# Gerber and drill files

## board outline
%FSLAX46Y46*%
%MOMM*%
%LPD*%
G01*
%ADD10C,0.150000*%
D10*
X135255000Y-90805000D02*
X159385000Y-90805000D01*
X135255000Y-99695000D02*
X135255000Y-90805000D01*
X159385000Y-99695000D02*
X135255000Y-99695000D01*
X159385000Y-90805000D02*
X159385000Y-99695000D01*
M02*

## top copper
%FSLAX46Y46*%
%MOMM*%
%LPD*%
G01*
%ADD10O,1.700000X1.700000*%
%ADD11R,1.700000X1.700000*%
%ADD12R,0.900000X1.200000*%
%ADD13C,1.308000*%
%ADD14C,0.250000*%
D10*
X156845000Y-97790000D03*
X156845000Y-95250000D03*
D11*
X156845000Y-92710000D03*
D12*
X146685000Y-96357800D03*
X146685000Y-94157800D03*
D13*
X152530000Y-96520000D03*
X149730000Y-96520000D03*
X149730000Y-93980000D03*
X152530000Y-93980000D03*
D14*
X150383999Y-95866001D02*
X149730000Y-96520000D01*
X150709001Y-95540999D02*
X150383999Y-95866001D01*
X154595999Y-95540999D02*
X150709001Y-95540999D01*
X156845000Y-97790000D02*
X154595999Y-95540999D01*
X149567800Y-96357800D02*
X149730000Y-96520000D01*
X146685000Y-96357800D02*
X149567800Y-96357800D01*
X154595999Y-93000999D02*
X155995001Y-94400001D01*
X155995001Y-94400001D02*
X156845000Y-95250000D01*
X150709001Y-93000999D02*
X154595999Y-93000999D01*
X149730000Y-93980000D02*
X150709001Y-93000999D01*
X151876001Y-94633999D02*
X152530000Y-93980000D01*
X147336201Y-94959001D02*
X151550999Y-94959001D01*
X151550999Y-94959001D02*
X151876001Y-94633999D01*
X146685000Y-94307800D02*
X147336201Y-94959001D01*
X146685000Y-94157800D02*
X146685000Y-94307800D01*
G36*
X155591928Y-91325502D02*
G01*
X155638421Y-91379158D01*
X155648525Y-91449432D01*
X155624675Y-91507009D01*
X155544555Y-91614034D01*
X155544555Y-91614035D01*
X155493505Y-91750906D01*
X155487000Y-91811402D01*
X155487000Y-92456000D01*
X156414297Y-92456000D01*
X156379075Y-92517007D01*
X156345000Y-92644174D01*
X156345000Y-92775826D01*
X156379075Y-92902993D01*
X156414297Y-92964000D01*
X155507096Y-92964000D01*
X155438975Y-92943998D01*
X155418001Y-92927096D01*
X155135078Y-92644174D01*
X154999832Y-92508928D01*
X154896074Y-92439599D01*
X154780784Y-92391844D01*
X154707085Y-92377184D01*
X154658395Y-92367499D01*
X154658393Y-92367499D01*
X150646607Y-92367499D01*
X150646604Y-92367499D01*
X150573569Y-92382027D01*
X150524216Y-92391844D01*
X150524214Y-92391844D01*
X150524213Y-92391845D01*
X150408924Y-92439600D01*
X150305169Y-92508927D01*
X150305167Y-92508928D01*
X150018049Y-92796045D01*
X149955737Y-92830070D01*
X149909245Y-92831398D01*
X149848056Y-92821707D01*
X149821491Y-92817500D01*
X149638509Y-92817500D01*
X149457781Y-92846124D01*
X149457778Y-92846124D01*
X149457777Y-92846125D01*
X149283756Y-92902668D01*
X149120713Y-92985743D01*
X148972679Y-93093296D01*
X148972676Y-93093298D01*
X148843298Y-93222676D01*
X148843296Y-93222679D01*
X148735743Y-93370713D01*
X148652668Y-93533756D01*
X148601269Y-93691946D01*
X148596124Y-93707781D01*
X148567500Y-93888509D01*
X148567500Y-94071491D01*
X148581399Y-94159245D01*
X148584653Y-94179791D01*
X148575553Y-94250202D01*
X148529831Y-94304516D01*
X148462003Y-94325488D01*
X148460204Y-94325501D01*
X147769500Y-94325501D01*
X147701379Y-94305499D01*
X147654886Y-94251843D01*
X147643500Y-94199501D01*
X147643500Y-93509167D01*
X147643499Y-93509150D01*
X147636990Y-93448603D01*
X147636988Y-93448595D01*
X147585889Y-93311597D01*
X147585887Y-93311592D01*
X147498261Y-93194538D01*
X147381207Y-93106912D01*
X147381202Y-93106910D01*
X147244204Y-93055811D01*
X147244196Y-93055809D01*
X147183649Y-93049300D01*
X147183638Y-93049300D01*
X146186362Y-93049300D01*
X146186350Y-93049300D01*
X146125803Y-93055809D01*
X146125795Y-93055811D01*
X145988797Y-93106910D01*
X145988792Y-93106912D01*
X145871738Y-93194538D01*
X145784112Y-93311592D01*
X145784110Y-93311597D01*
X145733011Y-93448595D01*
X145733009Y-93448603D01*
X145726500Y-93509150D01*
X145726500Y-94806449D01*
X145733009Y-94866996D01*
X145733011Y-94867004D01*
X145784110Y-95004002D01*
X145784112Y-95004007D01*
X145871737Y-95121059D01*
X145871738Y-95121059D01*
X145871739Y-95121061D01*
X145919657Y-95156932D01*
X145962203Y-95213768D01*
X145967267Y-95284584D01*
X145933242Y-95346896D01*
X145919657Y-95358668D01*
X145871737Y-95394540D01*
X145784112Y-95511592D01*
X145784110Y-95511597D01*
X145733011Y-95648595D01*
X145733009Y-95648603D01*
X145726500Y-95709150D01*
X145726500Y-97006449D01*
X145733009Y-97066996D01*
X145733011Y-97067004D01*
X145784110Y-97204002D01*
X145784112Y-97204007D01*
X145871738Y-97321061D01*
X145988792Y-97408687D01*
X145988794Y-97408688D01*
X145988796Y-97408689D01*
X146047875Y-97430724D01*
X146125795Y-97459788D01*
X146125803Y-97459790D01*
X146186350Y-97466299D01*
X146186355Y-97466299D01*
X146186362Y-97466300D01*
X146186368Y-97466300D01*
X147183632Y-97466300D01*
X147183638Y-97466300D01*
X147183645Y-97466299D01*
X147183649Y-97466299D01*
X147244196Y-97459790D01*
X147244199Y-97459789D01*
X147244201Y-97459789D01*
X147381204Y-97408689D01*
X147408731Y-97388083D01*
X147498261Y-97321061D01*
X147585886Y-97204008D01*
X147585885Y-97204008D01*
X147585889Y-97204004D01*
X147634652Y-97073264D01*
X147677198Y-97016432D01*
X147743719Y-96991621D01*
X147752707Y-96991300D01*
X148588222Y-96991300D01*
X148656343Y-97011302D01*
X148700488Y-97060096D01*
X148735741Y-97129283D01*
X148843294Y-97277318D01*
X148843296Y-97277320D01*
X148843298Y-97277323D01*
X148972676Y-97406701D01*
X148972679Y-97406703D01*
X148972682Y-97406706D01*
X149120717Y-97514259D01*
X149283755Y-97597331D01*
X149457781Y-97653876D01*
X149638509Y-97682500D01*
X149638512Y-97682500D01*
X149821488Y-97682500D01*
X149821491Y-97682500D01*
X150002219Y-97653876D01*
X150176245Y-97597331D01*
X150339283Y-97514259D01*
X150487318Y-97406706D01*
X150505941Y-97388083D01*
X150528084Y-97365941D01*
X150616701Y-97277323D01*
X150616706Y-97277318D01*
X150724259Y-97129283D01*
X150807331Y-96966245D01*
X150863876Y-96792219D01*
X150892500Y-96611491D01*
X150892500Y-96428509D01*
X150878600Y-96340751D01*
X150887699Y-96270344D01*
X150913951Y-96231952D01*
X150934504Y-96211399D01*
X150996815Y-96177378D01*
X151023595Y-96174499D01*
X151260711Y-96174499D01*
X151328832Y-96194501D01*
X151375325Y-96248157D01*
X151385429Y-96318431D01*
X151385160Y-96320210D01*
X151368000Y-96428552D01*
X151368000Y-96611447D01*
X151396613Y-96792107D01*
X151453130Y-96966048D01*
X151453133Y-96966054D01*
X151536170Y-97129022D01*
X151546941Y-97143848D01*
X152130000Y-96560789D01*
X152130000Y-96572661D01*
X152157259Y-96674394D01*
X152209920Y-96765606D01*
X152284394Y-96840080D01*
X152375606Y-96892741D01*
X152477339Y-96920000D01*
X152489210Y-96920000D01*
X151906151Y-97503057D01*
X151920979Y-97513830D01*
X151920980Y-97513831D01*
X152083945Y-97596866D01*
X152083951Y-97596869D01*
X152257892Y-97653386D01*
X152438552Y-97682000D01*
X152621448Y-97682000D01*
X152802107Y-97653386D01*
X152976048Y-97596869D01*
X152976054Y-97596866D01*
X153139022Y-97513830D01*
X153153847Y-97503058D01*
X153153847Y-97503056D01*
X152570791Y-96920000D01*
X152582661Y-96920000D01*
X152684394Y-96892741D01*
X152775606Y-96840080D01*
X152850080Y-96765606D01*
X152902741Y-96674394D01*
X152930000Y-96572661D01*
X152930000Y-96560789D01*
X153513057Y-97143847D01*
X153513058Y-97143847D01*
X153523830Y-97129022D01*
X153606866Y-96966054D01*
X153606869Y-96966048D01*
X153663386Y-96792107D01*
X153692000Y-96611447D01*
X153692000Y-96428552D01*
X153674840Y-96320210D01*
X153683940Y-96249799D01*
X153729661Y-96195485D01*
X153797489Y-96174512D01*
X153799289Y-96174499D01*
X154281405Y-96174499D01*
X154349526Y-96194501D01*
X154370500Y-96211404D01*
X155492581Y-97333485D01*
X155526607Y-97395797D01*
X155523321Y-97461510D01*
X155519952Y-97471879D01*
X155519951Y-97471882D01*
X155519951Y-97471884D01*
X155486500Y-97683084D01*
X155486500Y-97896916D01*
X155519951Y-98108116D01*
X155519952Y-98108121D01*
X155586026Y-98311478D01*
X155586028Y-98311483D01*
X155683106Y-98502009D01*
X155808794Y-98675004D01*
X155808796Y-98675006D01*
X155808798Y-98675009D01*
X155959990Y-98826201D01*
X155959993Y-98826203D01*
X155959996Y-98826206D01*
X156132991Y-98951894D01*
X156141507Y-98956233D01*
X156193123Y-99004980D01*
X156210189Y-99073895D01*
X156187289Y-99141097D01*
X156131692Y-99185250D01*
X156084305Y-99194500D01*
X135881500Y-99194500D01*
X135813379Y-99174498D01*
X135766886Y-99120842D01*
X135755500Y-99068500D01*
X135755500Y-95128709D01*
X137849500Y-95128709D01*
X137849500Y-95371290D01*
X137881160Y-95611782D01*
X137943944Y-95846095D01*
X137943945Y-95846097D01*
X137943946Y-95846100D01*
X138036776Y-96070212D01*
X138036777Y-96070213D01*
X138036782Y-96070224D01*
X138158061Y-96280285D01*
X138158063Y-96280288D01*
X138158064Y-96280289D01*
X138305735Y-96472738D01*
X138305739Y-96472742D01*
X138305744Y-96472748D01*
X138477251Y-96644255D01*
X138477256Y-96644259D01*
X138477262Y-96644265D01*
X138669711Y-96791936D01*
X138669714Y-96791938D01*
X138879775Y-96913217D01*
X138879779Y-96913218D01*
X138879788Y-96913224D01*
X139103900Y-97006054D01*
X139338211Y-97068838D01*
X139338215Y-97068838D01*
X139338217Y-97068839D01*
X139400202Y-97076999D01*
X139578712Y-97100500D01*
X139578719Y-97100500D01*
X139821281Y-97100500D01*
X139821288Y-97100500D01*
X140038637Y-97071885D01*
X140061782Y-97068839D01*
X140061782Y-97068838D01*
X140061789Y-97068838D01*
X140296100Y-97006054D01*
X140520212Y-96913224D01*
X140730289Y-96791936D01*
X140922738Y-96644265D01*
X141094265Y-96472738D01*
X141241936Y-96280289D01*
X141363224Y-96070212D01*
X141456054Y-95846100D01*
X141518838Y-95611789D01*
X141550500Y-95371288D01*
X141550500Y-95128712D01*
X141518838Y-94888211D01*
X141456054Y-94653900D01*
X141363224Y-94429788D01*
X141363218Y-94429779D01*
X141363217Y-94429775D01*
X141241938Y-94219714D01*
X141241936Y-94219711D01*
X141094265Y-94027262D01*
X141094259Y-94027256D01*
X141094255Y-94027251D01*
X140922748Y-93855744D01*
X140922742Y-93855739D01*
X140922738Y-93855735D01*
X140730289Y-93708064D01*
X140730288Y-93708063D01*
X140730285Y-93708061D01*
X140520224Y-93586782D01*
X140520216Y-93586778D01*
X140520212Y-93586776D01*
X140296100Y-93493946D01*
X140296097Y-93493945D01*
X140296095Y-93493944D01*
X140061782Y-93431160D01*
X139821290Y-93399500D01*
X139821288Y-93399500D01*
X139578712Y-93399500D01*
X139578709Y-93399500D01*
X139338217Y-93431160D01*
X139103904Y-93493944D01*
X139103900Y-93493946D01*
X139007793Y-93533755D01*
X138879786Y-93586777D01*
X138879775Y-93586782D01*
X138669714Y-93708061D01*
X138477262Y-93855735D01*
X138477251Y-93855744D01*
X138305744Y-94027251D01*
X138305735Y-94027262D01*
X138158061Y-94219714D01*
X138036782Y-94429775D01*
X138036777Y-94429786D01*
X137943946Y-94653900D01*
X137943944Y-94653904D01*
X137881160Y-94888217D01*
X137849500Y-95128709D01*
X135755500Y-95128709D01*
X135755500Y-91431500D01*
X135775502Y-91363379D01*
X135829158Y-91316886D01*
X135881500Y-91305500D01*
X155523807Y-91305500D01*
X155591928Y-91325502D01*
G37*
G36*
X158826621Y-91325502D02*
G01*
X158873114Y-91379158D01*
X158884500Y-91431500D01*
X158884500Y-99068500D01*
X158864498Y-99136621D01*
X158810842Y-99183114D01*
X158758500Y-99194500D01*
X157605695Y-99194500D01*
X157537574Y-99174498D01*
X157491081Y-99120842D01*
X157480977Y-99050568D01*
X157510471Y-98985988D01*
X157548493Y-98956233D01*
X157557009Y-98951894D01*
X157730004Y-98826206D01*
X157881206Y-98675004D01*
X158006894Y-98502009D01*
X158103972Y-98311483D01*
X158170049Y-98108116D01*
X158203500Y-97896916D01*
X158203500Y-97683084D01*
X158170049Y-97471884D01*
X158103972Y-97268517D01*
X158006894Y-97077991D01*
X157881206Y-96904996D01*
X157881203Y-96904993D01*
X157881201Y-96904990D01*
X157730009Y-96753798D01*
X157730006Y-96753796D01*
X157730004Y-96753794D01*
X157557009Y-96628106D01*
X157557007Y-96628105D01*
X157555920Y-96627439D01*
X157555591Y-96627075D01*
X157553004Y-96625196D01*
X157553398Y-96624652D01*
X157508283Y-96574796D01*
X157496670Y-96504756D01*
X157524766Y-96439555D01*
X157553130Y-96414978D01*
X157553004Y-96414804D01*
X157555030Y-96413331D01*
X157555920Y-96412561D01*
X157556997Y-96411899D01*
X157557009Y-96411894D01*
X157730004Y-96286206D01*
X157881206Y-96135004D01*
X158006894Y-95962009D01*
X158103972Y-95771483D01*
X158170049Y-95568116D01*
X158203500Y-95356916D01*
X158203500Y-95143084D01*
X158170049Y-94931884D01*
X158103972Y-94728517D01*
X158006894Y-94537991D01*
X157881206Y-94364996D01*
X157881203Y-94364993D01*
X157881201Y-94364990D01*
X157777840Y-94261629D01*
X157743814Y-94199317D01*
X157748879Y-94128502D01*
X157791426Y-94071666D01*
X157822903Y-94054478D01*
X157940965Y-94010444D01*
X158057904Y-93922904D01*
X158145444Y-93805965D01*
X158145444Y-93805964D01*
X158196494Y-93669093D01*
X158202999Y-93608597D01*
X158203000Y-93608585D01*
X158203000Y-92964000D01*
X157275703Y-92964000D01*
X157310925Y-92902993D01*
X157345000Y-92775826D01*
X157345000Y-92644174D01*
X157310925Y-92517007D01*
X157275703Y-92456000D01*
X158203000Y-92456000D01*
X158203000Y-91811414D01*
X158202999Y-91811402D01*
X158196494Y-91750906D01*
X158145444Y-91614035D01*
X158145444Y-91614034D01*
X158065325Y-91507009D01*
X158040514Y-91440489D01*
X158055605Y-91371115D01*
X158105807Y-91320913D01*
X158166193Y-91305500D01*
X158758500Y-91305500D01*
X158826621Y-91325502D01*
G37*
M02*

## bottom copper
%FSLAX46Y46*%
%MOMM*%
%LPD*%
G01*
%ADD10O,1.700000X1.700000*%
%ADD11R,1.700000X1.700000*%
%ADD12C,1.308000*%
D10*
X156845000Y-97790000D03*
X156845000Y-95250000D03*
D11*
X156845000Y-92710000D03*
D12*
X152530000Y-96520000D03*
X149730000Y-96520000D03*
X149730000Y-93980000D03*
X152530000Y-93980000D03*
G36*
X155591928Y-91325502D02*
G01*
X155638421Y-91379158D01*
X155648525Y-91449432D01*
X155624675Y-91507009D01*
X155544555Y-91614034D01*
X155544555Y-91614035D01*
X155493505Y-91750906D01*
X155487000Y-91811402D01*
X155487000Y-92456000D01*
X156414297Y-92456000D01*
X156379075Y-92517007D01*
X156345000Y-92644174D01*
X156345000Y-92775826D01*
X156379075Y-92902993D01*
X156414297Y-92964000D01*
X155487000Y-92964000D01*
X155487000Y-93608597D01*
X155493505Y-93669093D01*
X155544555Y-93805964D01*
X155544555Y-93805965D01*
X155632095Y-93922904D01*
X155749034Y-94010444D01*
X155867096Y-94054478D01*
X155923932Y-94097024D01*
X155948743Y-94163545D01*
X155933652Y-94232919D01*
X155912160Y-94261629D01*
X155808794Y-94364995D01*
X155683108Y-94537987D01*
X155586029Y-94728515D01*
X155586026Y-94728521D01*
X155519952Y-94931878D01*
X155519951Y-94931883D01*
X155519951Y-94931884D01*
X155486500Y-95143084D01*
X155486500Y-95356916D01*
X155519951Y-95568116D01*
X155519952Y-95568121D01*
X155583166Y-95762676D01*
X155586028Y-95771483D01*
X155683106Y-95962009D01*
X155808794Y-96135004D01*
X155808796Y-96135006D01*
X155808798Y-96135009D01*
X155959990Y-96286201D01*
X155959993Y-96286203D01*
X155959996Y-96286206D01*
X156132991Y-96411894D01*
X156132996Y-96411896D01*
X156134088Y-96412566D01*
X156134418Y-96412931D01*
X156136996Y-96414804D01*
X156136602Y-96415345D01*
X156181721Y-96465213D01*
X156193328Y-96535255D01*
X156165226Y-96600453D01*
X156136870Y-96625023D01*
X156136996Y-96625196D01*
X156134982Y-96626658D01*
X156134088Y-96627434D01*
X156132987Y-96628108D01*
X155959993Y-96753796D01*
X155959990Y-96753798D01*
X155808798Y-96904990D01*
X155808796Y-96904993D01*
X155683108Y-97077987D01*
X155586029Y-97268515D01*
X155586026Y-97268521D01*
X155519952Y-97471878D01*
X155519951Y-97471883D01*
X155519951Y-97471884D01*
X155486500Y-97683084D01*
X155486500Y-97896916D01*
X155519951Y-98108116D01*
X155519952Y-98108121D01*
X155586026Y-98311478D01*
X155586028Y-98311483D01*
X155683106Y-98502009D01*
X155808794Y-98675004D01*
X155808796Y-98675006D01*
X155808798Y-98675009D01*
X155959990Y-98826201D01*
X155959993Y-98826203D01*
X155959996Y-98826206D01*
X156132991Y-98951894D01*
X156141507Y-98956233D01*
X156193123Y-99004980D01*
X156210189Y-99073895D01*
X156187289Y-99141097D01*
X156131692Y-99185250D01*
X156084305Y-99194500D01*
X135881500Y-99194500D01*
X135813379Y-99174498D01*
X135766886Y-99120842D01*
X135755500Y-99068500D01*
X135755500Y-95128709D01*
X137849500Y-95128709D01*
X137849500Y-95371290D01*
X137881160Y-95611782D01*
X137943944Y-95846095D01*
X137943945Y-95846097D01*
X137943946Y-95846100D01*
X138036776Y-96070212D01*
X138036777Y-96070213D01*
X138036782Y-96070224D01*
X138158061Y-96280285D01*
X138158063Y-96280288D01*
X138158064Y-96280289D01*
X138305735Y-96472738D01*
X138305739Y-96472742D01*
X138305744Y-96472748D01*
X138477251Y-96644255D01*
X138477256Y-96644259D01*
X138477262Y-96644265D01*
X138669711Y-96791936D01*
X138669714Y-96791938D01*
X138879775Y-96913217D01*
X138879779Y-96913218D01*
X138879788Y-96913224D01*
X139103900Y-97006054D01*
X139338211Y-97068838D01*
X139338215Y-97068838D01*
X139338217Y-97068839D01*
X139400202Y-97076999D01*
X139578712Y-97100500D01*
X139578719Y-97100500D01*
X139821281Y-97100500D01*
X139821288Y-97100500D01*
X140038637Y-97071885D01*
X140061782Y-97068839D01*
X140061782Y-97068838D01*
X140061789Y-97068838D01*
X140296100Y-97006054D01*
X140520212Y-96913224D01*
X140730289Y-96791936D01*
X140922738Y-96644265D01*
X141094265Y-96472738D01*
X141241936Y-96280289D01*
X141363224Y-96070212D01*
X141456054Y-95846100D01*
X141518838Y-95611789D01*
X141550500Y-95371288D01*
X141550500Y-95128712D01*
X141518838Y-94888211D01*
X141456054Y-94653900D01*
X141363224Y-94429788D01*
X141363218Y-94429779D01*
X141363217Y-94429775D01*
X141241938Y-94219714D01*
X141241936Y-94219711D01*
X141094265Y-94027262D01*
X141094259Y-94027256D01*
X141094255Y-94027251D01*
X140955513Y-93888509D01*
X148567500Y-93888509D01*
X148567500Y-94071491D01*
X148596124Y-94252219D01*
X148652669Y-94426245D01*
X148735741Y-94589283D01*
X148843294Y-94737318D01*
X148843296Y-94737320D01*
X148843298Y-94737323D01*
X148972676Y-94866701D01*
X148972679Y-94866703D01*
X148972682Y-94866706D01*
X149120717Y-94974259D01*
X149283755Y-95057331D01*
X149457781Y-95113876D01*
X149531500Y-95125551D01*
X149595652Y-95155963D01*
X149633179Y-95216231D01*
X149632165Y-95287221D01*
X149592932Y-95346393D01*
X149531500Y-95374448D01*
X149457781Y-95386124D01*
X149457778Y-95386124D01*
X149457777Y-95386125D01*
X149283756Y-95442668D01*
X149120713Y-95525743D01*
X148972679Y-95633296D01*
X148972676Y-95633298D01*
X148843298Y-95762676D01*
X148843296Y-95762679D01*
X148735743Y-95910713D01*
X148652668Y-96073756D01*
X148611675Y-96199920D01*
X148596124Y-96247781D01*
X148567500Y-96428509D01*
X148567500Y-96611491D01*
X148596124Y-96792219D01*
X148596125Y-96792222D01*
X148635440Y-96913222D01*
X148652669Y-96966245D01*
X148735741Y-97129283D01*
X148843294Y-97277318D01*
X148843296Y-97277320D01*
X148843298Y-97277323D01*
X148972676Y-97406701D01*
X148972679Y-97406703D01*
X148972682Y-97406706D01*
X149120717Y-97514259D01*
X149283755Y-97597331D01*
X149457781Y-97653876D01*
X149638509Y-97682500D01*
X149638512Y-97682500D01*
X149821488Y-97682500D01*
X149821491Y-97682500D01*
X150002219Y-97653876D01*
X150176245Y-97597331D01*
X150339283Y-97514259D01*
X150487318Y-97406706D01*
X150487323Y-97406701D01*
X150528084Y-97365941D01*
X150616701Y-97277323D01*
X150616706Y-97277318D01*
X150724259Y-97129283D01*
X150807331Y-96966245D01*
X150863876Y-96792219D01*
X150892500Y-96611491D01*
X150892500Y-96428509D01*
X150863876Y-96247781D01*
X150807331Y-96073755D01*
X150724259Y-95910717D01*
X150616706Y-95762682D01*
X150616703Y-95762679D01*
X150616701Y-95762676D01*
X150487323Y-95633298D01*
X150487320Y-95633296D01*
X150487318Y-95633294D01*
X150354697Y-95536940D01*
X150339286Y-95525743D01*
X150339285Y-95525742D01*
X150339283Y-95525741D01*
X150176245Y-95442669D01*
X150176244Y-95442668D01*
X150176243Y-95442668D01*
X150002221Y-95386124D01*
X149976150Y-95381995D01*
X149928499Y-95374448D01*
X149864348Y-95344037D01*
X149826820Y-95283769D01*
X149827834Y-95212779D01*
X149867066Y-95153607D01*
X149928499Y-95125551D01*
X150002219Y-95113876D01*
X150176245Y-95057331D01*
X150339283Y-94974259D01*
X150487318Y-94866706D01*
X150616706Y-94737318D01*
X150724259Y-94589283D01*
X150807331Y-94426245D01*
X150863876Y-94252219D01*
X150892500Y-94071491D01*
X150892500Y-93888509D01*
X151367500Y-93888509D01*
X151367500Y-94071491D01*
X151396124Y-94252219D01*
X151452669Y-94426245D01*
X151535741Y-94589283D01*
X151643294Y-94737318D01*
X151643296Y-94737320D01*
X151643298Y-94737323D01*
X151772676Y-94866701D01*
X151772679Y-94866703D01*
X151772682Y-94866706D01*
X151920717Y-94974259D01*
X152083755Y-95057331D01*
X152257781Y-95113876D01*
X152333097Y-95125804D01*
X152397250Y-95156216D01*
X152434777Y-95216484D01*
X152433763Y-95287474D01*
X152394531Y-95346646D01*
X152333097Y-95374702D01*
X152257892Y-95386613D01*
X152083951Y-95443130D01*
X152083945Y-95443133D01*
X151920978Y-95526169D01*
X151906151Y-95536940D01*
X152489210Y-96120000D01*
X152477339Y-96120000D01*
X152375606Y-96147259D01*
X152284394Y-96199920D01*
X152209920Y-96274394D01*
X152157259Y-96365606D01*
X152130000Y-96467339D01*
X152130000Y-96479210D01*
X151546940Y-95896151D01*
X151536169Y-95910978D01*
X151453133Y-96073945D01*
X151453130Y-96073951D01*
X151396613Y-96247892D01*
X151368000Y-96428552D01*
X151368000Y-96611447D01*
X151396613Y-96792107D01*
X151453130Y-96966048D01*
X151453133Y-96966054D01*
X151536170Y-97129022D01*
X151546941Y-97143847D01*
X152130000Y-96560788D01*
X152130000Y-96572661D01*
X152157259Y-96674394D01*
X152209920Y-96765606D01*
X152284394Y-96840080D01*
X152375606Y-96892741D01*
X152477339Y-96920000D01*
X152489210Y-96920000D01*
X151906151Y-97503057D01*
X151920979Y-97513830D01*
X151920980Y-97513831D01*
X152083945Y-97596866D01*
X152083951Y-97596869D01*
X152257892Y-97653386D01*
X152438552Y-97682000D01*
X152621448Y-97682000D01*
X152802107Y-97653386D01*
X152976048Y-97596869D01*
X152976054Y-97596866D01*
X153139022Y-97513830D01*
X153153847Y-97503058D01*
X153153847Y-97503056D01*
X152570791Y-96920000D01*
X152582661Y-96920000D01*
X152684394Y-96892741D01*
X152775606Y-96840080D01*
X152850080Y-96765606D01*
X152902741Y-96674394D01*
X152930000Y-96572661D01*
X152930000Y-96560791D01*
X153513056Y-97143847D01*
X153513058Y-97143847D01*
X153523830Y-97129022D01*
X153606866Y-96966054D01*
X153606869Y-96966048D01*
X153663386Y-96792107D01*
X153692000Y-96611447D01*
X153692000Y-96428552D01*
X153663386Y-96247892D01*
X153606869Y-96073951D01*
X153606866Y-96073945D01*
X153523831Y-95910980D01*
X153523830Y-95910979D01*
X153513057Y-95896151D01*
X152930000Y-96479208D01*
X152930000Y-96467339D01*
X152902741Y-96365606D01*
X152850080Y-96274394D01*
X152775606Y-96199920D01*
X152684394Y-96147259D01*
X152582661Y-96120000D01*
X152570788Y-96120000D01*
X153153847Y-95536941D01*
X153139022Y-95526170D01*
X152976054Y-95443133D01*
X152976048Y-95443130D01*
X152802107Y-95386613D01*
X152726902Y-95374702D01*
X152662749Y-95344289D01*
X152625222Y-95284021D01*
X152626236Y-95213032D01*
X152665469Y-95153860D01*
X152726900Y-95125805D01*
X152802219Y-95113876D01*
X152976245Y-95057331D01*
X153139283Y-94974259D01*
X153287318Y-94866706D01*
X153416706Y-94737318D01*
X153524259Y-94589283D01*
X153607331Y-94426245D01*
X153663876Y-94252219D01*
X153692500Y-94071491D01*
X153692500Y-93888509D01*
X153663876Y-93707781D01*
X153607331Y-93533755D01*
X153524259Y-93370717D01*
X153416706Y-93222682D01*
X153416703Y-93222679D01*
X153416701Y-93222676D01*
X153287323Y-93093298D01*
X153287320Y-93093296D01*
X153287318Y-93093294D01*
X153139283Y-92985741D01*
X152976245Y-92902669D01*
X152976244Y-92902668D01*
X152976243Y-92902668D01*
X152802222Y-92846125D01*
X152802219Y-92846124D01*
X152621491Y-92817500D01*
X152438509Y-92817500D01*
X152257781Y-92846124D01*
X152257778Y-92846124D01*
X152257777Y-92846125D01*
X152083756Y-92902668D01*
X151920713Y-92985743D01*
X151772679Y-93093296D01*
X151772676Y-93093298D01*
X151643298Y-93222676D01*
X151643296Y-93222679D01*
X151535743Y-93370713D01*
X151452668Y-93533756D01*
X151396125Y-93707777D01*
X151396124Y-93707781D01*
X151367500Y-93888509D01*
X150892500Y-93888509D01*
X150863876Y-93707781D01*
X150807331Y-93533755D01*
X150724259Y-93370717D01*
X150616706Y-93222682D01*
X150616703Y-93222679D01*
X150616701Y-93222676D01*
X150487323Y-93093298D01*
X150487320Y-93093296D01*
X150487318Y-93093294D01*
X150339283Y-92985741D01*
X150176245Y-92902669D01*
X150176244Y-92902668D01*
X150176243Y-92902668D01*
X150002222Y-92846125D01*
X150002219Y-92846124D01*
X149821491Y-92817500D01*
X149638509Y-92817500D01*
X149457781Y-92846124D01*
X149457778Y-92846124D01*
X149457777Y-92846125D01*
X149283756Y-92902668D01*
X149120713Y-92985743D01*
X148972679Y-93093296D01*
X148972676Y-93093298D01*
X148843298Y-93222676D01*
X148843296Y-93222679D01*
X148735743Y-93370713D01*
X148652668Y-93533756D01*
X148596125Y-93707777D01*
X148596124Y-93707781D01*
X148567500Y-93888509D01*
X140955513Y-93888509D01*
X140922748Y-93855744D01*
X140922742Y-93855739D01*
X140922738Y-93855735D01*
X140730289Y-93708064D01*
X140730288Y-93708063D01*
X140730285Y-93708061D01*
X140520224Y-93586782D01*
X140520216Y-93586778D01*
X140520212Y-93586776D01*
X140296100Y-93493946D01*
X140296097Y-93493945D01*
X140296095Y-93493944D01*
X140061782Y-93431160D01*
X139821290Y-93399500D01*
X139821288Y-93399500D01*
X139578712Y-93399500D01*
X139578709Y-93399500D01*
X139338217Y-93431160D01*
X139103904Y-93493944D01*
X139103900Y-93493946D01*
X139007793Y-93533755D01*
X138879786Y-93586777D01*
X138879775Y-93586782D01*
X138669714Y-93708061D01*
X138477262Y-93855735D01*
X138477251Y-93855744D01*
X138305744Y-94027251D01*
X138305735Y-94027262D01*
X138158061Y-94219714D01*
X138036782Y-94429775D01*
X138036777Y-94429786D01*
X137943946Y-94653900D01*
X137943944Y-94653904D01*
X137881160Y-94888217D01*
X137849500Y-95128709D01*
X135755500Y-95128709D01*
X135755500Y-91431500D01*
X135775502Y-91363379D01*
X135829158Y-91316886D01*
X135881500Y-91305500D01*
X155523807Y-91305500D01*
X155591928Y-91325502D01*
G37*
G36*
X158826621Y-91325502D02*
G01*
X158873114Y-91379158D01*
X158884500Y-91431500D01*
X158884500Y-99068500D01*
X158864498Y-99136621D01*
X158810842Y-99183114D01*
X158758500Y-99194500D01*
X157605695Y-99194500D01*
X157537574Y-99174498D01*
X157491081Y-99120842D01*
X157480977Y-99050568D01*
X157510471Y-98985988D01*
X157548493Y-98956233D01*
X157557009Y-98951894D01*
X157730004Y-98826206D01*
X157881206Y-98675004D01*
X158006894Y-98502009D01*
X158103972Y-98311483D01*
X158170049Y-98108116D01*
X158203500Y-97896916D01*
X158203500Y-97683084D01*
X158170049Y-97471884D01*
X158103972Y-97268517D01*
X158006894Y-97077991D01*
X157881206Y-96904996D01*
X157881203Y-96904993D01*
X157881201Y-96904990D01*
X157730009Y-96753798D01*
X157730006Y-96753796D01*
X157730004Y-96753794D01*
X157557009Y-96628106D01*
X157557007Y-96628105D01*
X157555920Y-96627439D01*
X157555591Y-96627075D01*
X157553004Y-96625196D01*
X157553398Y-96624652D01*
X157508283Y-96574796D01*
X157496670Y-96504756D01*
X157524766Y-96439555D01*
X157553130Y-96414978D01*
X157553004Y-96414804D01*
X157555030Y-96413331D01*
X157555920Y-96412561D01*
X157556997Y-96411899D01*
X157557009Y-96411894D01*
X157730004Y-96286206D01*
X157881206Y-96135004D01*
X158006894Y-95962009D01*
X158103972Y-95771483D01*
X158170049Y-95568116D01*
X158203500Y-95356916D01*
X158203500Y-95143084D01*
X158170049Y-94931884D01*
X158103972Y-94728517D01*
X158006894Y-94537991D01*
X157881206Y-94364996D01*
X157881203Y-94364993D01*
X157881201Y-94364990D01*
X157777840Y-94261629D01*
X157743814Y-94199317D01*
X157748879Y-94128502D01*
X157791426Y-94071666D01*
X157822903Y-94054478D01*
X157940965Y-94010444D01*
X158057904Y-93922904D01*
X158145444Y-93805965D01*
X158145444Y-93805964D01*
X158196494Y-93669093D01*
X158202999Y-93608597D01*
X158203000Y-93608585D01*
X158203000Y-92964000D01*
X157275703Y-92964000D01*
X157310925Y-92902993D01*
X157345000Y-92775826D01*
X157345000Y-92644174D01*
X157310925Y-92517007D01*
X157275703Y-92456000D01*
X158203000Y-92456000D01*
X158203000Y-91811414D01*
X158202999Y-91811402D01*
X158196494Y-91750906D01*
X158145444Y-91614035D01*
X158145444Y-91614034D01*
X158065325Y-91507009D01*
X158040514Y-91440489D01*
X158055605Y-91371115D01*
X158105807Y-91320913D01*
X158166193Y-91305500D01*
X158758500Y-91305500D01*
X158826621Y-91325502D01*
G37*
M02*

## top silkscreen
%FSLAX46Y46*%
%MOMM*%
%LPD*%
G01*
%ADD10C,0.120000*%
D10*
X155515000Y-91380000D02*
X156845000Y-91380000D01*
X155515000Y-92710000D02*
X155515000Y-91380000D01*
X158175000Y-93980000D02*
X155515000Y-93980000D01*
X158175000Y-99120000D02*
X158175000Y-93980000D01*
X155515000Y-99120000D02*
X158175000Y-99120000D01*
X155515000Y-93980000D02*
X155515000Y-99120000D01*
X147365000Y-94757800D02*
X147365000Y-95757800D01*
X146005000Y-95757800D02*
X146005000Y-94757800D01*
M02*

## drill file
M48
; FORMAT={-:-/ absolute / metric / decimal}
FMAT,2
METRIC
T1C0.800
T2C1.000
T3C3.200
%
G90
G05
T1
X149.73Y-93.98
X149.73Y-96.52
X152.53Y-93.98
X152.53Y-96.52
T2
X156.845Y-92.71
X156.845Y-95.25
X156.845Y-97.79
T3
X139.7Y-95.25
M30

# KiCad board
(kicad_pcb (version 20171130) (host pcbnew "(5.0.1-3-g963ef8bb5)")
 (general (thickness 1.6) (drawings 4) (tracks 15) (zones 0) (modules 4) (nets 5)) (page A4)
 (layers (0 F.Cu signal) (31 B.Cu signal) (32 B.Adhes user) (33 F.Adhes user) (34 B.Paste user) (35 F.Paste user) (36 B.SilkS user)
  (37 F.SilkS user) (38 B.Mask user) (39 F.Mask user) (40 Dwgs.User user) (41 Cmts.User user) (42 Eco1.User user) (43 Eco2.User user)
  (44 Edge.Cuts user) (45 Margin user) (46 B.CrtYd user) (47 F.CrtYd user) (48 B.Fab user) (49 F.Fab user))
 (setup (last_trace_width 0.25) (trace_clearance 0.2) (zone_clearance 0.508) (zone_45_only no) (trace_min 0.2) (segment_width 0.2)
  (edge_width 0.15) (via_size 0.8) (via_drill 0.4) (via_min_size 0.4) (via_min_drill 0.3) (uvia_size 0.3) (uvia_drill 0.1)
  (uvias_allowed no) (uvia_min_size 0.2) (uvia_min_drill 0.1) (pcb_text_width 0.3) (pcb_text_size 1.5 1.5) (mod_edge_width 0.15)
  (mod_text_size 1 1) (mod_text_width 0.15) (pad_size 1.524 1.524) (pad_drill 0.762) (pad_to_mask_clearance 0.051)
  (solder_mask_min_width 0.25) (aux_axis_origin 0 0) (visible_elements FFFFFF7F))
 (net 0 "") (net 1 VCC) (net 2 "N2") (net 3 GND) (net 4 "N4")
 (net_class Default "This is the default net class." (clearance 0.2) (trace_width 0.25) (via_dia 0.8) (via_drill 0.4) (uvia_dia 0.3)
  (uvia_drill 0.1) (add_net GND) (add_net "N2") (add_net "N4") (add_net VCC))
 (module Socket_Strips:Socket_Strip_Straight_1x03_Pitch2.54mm (layer F.Cu) (at 156.845 92.71)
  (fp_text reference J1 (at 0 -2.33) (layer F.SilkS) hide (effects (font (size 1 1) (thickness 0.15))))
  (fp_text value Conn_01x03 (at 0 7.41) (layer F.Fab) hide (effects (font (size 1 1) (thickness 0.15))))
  (fp_line (start -1.33 -1.33) (end 0 -1.33) (layer F.SilkS) (width 0.12))
  (fp_line (start -1.33 0) (end -1.33 -1.33) (layer F.SilkS) (width 0.12))
  (fp_line (start 1.33 1.27) (end -1.33 1.27) (layer F.SilkS) (width 0.12))
  (fp_line (start 1.33 6.41) (end 1.33 1.27) (layer F.SilkS) (width 0.12))
  (fp_line (start -1.33 6.41) (end 1.33 6.41) (layer F.SilkS) (width 0.12))
  (fp_line (start -1.33 1.27) (end -1.33 6.41) (layer F.SilkS) (width 0.12))
  (pad 3 thru_hole oval (at 0 5.08) (size 1.7 1.7) (drill 1) (layers *.Cu *.Mask) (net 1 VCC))
  (pad 2 thru_hole oval (at 0 2.54) (size 1.7 1.7) (drill 1) (layers *.Cu *.Mask) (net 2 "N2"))
  (pad 1 thru_hole rect (at 0 0) (size 1.7 1.7) (drill 1) (layers *.Cu *.Mask) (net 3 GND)))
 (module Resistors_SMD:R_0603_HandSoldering (layer F.Cu) (at 146.685 95.2578 90)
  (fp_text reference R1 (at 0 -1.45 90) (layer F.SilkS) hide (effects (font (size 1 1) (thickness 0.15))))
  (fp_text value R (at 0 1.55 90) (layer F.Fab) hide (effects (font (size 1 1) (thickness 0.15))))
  (fp_line (start 0.5 0.68) (end -0.5 0.68) (layer F.SilkS) (width 0.12))
  (fp_line (start -0.5 -0.68) (end 0.5 -0.68) (layer F.SilkS) (width 0.12))
  (pad 1 smd rect (at -1.1 0 90) (size 1.2 0.9) (layers F.Cu F.Paste F.Mask) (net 1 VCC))
  (pad 2 smd rect (at 1.1 0 90) (size 1.2 0.9) (layers F.Cu F.Paste F.Mask) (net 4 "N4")))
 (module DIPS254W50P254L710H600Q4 (layer B.Cu) (at 151.13 95.25 180)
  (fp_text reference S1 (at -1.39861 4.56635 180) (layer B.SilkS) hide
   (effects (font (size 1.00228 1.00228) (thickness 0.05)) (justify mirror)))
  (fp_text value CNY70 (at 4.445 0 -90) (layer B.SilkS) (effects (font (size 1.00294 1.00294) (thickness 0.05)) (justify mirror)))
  (pad CATH thru_hole circle (at -1.4 -1.27 180) (size 1.308 1.308) (drill 0.8) (layers *.Cu *.Mask) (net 3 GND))
  (pad COLL thru_hole circle (at 1.4 -1.27 180) (size 1.308 1.308) (drill 0.8) (layers *.Cu *.Mask) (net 1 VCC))
  (pad E thru_hole circle (at 1.4 1.27 180) (size 1.308 1.308) (drill 0.8) (layers *.Cu *.Mask) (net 2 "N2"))
  (pad A thru_hole circle (at -1.4 1.27 180) (size 1.308 1.308) (drill 0.8) (layers *.Cu *.Mask) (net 4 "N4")))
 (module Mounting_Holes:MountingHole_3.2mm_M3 (layer F.Cu) (at 139.7 95.25)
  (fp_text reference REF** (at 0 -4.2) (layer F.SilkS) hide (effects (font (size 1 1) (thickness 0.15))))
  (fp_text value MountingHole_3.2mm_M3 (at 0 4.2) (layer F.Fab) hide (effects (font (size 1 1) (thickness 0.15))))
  (pad 1 np_thru_hole circle (at 0 0) (size 3.2 3.2) (drill 3.2) (layers *.Cu *.Mask)))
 (gr_line (start 135.255 90.805) (end 159.385 90.805) (layer Edge.Cuts) (width 0.15))
 (gr_line (start 135.255 99.695) (end 135.255 90.805) (layer Edge.Cuts) (width 0.15))
 (gr_line (start 159.385 99.695) (end 135.255 99.695) (layer Edge.Cuts) (width 0.15))
 (gr_line (start 159.385 90.805) (end 159.385 99.695) (layer Edge.Cuts) (width 0.15))
 (segment (start 150.383999 95.866001) (end 149.73 96.52) (width 0.25) (layer F.Cu) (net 1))
 (segment (start 150.709001 95.540999) (end 150.383999 95.866001) (width 0.25) (layer F.Cu) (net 1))
 (segment (start 154.595999 95.540999) (end 150.709001 95.540999) (width 0.25) (layer F.Cu) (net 1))
 (segment (start 156.845 97.79) (end 154.595999 95.540999) (width 0.25) (layer F.Cu) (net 1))
 (segment (start 149.5678 96.3578) (end 149.73 96.52) (width 0.25) (layer F.Cu) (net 1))
 (segment (start 146.685 96.3578) (end 149.5678 96.3578) (width 0.25) (layer F.Cu) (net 1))
 (segment (start 154.595999 93.000999) (end 155.995001 94.400001) (width 0.25) (layer F.Cu) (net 2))
 (segment (start 155.995001 94.400001) (end 156.845 95.25) (width 0.25) (layer F.Cu) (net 2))
 (segment (start 150.709001 93.000999) (end 154.595999 93.000999) (width 0.25) (layer F.Cu) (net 2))
 (segment (start 149.73 93.98) (end 150.709001 93.000999) (width 0.25) (layer F.Cu) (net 2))
 (segment (start 151.876001 94.633999) (end 152.53 93.98) (width 0.25) (layer F.Cu) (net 4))
 (segment (start 147.336201 94.959001) (end 151.550999 94.959001) (width 0.25) (layer F.Cu) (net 4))
 (segment (start 151.550999 94.959001) (end 151.876001 94.633999) (width 0.25) (layer F.Cu) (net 4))
 (segment (start 146.685 94.3078) (end 147.336201 94.959001) (width 0.25) (layer F.Cu) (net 4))
 (segment (start 146.685 94.1578) (end 146.685 94.3078) (width 0.25) (layer F.Cu) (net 4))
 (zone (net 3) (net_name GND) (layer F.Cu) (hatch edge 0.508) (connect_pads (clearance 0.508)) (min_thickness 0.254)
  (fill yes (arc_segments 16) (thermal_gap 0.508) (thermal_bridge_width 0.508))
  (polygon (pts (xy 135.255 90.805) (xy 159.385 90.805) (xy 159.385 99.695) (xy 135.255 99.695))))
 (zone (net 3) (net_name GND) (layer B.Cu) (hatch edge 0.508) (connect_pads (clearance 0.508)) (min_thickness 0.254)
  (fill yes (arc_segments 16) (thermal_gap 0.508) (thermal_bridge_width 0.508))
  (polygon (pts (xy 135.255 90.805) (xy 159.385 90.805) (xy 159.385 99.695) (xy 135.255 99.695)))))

